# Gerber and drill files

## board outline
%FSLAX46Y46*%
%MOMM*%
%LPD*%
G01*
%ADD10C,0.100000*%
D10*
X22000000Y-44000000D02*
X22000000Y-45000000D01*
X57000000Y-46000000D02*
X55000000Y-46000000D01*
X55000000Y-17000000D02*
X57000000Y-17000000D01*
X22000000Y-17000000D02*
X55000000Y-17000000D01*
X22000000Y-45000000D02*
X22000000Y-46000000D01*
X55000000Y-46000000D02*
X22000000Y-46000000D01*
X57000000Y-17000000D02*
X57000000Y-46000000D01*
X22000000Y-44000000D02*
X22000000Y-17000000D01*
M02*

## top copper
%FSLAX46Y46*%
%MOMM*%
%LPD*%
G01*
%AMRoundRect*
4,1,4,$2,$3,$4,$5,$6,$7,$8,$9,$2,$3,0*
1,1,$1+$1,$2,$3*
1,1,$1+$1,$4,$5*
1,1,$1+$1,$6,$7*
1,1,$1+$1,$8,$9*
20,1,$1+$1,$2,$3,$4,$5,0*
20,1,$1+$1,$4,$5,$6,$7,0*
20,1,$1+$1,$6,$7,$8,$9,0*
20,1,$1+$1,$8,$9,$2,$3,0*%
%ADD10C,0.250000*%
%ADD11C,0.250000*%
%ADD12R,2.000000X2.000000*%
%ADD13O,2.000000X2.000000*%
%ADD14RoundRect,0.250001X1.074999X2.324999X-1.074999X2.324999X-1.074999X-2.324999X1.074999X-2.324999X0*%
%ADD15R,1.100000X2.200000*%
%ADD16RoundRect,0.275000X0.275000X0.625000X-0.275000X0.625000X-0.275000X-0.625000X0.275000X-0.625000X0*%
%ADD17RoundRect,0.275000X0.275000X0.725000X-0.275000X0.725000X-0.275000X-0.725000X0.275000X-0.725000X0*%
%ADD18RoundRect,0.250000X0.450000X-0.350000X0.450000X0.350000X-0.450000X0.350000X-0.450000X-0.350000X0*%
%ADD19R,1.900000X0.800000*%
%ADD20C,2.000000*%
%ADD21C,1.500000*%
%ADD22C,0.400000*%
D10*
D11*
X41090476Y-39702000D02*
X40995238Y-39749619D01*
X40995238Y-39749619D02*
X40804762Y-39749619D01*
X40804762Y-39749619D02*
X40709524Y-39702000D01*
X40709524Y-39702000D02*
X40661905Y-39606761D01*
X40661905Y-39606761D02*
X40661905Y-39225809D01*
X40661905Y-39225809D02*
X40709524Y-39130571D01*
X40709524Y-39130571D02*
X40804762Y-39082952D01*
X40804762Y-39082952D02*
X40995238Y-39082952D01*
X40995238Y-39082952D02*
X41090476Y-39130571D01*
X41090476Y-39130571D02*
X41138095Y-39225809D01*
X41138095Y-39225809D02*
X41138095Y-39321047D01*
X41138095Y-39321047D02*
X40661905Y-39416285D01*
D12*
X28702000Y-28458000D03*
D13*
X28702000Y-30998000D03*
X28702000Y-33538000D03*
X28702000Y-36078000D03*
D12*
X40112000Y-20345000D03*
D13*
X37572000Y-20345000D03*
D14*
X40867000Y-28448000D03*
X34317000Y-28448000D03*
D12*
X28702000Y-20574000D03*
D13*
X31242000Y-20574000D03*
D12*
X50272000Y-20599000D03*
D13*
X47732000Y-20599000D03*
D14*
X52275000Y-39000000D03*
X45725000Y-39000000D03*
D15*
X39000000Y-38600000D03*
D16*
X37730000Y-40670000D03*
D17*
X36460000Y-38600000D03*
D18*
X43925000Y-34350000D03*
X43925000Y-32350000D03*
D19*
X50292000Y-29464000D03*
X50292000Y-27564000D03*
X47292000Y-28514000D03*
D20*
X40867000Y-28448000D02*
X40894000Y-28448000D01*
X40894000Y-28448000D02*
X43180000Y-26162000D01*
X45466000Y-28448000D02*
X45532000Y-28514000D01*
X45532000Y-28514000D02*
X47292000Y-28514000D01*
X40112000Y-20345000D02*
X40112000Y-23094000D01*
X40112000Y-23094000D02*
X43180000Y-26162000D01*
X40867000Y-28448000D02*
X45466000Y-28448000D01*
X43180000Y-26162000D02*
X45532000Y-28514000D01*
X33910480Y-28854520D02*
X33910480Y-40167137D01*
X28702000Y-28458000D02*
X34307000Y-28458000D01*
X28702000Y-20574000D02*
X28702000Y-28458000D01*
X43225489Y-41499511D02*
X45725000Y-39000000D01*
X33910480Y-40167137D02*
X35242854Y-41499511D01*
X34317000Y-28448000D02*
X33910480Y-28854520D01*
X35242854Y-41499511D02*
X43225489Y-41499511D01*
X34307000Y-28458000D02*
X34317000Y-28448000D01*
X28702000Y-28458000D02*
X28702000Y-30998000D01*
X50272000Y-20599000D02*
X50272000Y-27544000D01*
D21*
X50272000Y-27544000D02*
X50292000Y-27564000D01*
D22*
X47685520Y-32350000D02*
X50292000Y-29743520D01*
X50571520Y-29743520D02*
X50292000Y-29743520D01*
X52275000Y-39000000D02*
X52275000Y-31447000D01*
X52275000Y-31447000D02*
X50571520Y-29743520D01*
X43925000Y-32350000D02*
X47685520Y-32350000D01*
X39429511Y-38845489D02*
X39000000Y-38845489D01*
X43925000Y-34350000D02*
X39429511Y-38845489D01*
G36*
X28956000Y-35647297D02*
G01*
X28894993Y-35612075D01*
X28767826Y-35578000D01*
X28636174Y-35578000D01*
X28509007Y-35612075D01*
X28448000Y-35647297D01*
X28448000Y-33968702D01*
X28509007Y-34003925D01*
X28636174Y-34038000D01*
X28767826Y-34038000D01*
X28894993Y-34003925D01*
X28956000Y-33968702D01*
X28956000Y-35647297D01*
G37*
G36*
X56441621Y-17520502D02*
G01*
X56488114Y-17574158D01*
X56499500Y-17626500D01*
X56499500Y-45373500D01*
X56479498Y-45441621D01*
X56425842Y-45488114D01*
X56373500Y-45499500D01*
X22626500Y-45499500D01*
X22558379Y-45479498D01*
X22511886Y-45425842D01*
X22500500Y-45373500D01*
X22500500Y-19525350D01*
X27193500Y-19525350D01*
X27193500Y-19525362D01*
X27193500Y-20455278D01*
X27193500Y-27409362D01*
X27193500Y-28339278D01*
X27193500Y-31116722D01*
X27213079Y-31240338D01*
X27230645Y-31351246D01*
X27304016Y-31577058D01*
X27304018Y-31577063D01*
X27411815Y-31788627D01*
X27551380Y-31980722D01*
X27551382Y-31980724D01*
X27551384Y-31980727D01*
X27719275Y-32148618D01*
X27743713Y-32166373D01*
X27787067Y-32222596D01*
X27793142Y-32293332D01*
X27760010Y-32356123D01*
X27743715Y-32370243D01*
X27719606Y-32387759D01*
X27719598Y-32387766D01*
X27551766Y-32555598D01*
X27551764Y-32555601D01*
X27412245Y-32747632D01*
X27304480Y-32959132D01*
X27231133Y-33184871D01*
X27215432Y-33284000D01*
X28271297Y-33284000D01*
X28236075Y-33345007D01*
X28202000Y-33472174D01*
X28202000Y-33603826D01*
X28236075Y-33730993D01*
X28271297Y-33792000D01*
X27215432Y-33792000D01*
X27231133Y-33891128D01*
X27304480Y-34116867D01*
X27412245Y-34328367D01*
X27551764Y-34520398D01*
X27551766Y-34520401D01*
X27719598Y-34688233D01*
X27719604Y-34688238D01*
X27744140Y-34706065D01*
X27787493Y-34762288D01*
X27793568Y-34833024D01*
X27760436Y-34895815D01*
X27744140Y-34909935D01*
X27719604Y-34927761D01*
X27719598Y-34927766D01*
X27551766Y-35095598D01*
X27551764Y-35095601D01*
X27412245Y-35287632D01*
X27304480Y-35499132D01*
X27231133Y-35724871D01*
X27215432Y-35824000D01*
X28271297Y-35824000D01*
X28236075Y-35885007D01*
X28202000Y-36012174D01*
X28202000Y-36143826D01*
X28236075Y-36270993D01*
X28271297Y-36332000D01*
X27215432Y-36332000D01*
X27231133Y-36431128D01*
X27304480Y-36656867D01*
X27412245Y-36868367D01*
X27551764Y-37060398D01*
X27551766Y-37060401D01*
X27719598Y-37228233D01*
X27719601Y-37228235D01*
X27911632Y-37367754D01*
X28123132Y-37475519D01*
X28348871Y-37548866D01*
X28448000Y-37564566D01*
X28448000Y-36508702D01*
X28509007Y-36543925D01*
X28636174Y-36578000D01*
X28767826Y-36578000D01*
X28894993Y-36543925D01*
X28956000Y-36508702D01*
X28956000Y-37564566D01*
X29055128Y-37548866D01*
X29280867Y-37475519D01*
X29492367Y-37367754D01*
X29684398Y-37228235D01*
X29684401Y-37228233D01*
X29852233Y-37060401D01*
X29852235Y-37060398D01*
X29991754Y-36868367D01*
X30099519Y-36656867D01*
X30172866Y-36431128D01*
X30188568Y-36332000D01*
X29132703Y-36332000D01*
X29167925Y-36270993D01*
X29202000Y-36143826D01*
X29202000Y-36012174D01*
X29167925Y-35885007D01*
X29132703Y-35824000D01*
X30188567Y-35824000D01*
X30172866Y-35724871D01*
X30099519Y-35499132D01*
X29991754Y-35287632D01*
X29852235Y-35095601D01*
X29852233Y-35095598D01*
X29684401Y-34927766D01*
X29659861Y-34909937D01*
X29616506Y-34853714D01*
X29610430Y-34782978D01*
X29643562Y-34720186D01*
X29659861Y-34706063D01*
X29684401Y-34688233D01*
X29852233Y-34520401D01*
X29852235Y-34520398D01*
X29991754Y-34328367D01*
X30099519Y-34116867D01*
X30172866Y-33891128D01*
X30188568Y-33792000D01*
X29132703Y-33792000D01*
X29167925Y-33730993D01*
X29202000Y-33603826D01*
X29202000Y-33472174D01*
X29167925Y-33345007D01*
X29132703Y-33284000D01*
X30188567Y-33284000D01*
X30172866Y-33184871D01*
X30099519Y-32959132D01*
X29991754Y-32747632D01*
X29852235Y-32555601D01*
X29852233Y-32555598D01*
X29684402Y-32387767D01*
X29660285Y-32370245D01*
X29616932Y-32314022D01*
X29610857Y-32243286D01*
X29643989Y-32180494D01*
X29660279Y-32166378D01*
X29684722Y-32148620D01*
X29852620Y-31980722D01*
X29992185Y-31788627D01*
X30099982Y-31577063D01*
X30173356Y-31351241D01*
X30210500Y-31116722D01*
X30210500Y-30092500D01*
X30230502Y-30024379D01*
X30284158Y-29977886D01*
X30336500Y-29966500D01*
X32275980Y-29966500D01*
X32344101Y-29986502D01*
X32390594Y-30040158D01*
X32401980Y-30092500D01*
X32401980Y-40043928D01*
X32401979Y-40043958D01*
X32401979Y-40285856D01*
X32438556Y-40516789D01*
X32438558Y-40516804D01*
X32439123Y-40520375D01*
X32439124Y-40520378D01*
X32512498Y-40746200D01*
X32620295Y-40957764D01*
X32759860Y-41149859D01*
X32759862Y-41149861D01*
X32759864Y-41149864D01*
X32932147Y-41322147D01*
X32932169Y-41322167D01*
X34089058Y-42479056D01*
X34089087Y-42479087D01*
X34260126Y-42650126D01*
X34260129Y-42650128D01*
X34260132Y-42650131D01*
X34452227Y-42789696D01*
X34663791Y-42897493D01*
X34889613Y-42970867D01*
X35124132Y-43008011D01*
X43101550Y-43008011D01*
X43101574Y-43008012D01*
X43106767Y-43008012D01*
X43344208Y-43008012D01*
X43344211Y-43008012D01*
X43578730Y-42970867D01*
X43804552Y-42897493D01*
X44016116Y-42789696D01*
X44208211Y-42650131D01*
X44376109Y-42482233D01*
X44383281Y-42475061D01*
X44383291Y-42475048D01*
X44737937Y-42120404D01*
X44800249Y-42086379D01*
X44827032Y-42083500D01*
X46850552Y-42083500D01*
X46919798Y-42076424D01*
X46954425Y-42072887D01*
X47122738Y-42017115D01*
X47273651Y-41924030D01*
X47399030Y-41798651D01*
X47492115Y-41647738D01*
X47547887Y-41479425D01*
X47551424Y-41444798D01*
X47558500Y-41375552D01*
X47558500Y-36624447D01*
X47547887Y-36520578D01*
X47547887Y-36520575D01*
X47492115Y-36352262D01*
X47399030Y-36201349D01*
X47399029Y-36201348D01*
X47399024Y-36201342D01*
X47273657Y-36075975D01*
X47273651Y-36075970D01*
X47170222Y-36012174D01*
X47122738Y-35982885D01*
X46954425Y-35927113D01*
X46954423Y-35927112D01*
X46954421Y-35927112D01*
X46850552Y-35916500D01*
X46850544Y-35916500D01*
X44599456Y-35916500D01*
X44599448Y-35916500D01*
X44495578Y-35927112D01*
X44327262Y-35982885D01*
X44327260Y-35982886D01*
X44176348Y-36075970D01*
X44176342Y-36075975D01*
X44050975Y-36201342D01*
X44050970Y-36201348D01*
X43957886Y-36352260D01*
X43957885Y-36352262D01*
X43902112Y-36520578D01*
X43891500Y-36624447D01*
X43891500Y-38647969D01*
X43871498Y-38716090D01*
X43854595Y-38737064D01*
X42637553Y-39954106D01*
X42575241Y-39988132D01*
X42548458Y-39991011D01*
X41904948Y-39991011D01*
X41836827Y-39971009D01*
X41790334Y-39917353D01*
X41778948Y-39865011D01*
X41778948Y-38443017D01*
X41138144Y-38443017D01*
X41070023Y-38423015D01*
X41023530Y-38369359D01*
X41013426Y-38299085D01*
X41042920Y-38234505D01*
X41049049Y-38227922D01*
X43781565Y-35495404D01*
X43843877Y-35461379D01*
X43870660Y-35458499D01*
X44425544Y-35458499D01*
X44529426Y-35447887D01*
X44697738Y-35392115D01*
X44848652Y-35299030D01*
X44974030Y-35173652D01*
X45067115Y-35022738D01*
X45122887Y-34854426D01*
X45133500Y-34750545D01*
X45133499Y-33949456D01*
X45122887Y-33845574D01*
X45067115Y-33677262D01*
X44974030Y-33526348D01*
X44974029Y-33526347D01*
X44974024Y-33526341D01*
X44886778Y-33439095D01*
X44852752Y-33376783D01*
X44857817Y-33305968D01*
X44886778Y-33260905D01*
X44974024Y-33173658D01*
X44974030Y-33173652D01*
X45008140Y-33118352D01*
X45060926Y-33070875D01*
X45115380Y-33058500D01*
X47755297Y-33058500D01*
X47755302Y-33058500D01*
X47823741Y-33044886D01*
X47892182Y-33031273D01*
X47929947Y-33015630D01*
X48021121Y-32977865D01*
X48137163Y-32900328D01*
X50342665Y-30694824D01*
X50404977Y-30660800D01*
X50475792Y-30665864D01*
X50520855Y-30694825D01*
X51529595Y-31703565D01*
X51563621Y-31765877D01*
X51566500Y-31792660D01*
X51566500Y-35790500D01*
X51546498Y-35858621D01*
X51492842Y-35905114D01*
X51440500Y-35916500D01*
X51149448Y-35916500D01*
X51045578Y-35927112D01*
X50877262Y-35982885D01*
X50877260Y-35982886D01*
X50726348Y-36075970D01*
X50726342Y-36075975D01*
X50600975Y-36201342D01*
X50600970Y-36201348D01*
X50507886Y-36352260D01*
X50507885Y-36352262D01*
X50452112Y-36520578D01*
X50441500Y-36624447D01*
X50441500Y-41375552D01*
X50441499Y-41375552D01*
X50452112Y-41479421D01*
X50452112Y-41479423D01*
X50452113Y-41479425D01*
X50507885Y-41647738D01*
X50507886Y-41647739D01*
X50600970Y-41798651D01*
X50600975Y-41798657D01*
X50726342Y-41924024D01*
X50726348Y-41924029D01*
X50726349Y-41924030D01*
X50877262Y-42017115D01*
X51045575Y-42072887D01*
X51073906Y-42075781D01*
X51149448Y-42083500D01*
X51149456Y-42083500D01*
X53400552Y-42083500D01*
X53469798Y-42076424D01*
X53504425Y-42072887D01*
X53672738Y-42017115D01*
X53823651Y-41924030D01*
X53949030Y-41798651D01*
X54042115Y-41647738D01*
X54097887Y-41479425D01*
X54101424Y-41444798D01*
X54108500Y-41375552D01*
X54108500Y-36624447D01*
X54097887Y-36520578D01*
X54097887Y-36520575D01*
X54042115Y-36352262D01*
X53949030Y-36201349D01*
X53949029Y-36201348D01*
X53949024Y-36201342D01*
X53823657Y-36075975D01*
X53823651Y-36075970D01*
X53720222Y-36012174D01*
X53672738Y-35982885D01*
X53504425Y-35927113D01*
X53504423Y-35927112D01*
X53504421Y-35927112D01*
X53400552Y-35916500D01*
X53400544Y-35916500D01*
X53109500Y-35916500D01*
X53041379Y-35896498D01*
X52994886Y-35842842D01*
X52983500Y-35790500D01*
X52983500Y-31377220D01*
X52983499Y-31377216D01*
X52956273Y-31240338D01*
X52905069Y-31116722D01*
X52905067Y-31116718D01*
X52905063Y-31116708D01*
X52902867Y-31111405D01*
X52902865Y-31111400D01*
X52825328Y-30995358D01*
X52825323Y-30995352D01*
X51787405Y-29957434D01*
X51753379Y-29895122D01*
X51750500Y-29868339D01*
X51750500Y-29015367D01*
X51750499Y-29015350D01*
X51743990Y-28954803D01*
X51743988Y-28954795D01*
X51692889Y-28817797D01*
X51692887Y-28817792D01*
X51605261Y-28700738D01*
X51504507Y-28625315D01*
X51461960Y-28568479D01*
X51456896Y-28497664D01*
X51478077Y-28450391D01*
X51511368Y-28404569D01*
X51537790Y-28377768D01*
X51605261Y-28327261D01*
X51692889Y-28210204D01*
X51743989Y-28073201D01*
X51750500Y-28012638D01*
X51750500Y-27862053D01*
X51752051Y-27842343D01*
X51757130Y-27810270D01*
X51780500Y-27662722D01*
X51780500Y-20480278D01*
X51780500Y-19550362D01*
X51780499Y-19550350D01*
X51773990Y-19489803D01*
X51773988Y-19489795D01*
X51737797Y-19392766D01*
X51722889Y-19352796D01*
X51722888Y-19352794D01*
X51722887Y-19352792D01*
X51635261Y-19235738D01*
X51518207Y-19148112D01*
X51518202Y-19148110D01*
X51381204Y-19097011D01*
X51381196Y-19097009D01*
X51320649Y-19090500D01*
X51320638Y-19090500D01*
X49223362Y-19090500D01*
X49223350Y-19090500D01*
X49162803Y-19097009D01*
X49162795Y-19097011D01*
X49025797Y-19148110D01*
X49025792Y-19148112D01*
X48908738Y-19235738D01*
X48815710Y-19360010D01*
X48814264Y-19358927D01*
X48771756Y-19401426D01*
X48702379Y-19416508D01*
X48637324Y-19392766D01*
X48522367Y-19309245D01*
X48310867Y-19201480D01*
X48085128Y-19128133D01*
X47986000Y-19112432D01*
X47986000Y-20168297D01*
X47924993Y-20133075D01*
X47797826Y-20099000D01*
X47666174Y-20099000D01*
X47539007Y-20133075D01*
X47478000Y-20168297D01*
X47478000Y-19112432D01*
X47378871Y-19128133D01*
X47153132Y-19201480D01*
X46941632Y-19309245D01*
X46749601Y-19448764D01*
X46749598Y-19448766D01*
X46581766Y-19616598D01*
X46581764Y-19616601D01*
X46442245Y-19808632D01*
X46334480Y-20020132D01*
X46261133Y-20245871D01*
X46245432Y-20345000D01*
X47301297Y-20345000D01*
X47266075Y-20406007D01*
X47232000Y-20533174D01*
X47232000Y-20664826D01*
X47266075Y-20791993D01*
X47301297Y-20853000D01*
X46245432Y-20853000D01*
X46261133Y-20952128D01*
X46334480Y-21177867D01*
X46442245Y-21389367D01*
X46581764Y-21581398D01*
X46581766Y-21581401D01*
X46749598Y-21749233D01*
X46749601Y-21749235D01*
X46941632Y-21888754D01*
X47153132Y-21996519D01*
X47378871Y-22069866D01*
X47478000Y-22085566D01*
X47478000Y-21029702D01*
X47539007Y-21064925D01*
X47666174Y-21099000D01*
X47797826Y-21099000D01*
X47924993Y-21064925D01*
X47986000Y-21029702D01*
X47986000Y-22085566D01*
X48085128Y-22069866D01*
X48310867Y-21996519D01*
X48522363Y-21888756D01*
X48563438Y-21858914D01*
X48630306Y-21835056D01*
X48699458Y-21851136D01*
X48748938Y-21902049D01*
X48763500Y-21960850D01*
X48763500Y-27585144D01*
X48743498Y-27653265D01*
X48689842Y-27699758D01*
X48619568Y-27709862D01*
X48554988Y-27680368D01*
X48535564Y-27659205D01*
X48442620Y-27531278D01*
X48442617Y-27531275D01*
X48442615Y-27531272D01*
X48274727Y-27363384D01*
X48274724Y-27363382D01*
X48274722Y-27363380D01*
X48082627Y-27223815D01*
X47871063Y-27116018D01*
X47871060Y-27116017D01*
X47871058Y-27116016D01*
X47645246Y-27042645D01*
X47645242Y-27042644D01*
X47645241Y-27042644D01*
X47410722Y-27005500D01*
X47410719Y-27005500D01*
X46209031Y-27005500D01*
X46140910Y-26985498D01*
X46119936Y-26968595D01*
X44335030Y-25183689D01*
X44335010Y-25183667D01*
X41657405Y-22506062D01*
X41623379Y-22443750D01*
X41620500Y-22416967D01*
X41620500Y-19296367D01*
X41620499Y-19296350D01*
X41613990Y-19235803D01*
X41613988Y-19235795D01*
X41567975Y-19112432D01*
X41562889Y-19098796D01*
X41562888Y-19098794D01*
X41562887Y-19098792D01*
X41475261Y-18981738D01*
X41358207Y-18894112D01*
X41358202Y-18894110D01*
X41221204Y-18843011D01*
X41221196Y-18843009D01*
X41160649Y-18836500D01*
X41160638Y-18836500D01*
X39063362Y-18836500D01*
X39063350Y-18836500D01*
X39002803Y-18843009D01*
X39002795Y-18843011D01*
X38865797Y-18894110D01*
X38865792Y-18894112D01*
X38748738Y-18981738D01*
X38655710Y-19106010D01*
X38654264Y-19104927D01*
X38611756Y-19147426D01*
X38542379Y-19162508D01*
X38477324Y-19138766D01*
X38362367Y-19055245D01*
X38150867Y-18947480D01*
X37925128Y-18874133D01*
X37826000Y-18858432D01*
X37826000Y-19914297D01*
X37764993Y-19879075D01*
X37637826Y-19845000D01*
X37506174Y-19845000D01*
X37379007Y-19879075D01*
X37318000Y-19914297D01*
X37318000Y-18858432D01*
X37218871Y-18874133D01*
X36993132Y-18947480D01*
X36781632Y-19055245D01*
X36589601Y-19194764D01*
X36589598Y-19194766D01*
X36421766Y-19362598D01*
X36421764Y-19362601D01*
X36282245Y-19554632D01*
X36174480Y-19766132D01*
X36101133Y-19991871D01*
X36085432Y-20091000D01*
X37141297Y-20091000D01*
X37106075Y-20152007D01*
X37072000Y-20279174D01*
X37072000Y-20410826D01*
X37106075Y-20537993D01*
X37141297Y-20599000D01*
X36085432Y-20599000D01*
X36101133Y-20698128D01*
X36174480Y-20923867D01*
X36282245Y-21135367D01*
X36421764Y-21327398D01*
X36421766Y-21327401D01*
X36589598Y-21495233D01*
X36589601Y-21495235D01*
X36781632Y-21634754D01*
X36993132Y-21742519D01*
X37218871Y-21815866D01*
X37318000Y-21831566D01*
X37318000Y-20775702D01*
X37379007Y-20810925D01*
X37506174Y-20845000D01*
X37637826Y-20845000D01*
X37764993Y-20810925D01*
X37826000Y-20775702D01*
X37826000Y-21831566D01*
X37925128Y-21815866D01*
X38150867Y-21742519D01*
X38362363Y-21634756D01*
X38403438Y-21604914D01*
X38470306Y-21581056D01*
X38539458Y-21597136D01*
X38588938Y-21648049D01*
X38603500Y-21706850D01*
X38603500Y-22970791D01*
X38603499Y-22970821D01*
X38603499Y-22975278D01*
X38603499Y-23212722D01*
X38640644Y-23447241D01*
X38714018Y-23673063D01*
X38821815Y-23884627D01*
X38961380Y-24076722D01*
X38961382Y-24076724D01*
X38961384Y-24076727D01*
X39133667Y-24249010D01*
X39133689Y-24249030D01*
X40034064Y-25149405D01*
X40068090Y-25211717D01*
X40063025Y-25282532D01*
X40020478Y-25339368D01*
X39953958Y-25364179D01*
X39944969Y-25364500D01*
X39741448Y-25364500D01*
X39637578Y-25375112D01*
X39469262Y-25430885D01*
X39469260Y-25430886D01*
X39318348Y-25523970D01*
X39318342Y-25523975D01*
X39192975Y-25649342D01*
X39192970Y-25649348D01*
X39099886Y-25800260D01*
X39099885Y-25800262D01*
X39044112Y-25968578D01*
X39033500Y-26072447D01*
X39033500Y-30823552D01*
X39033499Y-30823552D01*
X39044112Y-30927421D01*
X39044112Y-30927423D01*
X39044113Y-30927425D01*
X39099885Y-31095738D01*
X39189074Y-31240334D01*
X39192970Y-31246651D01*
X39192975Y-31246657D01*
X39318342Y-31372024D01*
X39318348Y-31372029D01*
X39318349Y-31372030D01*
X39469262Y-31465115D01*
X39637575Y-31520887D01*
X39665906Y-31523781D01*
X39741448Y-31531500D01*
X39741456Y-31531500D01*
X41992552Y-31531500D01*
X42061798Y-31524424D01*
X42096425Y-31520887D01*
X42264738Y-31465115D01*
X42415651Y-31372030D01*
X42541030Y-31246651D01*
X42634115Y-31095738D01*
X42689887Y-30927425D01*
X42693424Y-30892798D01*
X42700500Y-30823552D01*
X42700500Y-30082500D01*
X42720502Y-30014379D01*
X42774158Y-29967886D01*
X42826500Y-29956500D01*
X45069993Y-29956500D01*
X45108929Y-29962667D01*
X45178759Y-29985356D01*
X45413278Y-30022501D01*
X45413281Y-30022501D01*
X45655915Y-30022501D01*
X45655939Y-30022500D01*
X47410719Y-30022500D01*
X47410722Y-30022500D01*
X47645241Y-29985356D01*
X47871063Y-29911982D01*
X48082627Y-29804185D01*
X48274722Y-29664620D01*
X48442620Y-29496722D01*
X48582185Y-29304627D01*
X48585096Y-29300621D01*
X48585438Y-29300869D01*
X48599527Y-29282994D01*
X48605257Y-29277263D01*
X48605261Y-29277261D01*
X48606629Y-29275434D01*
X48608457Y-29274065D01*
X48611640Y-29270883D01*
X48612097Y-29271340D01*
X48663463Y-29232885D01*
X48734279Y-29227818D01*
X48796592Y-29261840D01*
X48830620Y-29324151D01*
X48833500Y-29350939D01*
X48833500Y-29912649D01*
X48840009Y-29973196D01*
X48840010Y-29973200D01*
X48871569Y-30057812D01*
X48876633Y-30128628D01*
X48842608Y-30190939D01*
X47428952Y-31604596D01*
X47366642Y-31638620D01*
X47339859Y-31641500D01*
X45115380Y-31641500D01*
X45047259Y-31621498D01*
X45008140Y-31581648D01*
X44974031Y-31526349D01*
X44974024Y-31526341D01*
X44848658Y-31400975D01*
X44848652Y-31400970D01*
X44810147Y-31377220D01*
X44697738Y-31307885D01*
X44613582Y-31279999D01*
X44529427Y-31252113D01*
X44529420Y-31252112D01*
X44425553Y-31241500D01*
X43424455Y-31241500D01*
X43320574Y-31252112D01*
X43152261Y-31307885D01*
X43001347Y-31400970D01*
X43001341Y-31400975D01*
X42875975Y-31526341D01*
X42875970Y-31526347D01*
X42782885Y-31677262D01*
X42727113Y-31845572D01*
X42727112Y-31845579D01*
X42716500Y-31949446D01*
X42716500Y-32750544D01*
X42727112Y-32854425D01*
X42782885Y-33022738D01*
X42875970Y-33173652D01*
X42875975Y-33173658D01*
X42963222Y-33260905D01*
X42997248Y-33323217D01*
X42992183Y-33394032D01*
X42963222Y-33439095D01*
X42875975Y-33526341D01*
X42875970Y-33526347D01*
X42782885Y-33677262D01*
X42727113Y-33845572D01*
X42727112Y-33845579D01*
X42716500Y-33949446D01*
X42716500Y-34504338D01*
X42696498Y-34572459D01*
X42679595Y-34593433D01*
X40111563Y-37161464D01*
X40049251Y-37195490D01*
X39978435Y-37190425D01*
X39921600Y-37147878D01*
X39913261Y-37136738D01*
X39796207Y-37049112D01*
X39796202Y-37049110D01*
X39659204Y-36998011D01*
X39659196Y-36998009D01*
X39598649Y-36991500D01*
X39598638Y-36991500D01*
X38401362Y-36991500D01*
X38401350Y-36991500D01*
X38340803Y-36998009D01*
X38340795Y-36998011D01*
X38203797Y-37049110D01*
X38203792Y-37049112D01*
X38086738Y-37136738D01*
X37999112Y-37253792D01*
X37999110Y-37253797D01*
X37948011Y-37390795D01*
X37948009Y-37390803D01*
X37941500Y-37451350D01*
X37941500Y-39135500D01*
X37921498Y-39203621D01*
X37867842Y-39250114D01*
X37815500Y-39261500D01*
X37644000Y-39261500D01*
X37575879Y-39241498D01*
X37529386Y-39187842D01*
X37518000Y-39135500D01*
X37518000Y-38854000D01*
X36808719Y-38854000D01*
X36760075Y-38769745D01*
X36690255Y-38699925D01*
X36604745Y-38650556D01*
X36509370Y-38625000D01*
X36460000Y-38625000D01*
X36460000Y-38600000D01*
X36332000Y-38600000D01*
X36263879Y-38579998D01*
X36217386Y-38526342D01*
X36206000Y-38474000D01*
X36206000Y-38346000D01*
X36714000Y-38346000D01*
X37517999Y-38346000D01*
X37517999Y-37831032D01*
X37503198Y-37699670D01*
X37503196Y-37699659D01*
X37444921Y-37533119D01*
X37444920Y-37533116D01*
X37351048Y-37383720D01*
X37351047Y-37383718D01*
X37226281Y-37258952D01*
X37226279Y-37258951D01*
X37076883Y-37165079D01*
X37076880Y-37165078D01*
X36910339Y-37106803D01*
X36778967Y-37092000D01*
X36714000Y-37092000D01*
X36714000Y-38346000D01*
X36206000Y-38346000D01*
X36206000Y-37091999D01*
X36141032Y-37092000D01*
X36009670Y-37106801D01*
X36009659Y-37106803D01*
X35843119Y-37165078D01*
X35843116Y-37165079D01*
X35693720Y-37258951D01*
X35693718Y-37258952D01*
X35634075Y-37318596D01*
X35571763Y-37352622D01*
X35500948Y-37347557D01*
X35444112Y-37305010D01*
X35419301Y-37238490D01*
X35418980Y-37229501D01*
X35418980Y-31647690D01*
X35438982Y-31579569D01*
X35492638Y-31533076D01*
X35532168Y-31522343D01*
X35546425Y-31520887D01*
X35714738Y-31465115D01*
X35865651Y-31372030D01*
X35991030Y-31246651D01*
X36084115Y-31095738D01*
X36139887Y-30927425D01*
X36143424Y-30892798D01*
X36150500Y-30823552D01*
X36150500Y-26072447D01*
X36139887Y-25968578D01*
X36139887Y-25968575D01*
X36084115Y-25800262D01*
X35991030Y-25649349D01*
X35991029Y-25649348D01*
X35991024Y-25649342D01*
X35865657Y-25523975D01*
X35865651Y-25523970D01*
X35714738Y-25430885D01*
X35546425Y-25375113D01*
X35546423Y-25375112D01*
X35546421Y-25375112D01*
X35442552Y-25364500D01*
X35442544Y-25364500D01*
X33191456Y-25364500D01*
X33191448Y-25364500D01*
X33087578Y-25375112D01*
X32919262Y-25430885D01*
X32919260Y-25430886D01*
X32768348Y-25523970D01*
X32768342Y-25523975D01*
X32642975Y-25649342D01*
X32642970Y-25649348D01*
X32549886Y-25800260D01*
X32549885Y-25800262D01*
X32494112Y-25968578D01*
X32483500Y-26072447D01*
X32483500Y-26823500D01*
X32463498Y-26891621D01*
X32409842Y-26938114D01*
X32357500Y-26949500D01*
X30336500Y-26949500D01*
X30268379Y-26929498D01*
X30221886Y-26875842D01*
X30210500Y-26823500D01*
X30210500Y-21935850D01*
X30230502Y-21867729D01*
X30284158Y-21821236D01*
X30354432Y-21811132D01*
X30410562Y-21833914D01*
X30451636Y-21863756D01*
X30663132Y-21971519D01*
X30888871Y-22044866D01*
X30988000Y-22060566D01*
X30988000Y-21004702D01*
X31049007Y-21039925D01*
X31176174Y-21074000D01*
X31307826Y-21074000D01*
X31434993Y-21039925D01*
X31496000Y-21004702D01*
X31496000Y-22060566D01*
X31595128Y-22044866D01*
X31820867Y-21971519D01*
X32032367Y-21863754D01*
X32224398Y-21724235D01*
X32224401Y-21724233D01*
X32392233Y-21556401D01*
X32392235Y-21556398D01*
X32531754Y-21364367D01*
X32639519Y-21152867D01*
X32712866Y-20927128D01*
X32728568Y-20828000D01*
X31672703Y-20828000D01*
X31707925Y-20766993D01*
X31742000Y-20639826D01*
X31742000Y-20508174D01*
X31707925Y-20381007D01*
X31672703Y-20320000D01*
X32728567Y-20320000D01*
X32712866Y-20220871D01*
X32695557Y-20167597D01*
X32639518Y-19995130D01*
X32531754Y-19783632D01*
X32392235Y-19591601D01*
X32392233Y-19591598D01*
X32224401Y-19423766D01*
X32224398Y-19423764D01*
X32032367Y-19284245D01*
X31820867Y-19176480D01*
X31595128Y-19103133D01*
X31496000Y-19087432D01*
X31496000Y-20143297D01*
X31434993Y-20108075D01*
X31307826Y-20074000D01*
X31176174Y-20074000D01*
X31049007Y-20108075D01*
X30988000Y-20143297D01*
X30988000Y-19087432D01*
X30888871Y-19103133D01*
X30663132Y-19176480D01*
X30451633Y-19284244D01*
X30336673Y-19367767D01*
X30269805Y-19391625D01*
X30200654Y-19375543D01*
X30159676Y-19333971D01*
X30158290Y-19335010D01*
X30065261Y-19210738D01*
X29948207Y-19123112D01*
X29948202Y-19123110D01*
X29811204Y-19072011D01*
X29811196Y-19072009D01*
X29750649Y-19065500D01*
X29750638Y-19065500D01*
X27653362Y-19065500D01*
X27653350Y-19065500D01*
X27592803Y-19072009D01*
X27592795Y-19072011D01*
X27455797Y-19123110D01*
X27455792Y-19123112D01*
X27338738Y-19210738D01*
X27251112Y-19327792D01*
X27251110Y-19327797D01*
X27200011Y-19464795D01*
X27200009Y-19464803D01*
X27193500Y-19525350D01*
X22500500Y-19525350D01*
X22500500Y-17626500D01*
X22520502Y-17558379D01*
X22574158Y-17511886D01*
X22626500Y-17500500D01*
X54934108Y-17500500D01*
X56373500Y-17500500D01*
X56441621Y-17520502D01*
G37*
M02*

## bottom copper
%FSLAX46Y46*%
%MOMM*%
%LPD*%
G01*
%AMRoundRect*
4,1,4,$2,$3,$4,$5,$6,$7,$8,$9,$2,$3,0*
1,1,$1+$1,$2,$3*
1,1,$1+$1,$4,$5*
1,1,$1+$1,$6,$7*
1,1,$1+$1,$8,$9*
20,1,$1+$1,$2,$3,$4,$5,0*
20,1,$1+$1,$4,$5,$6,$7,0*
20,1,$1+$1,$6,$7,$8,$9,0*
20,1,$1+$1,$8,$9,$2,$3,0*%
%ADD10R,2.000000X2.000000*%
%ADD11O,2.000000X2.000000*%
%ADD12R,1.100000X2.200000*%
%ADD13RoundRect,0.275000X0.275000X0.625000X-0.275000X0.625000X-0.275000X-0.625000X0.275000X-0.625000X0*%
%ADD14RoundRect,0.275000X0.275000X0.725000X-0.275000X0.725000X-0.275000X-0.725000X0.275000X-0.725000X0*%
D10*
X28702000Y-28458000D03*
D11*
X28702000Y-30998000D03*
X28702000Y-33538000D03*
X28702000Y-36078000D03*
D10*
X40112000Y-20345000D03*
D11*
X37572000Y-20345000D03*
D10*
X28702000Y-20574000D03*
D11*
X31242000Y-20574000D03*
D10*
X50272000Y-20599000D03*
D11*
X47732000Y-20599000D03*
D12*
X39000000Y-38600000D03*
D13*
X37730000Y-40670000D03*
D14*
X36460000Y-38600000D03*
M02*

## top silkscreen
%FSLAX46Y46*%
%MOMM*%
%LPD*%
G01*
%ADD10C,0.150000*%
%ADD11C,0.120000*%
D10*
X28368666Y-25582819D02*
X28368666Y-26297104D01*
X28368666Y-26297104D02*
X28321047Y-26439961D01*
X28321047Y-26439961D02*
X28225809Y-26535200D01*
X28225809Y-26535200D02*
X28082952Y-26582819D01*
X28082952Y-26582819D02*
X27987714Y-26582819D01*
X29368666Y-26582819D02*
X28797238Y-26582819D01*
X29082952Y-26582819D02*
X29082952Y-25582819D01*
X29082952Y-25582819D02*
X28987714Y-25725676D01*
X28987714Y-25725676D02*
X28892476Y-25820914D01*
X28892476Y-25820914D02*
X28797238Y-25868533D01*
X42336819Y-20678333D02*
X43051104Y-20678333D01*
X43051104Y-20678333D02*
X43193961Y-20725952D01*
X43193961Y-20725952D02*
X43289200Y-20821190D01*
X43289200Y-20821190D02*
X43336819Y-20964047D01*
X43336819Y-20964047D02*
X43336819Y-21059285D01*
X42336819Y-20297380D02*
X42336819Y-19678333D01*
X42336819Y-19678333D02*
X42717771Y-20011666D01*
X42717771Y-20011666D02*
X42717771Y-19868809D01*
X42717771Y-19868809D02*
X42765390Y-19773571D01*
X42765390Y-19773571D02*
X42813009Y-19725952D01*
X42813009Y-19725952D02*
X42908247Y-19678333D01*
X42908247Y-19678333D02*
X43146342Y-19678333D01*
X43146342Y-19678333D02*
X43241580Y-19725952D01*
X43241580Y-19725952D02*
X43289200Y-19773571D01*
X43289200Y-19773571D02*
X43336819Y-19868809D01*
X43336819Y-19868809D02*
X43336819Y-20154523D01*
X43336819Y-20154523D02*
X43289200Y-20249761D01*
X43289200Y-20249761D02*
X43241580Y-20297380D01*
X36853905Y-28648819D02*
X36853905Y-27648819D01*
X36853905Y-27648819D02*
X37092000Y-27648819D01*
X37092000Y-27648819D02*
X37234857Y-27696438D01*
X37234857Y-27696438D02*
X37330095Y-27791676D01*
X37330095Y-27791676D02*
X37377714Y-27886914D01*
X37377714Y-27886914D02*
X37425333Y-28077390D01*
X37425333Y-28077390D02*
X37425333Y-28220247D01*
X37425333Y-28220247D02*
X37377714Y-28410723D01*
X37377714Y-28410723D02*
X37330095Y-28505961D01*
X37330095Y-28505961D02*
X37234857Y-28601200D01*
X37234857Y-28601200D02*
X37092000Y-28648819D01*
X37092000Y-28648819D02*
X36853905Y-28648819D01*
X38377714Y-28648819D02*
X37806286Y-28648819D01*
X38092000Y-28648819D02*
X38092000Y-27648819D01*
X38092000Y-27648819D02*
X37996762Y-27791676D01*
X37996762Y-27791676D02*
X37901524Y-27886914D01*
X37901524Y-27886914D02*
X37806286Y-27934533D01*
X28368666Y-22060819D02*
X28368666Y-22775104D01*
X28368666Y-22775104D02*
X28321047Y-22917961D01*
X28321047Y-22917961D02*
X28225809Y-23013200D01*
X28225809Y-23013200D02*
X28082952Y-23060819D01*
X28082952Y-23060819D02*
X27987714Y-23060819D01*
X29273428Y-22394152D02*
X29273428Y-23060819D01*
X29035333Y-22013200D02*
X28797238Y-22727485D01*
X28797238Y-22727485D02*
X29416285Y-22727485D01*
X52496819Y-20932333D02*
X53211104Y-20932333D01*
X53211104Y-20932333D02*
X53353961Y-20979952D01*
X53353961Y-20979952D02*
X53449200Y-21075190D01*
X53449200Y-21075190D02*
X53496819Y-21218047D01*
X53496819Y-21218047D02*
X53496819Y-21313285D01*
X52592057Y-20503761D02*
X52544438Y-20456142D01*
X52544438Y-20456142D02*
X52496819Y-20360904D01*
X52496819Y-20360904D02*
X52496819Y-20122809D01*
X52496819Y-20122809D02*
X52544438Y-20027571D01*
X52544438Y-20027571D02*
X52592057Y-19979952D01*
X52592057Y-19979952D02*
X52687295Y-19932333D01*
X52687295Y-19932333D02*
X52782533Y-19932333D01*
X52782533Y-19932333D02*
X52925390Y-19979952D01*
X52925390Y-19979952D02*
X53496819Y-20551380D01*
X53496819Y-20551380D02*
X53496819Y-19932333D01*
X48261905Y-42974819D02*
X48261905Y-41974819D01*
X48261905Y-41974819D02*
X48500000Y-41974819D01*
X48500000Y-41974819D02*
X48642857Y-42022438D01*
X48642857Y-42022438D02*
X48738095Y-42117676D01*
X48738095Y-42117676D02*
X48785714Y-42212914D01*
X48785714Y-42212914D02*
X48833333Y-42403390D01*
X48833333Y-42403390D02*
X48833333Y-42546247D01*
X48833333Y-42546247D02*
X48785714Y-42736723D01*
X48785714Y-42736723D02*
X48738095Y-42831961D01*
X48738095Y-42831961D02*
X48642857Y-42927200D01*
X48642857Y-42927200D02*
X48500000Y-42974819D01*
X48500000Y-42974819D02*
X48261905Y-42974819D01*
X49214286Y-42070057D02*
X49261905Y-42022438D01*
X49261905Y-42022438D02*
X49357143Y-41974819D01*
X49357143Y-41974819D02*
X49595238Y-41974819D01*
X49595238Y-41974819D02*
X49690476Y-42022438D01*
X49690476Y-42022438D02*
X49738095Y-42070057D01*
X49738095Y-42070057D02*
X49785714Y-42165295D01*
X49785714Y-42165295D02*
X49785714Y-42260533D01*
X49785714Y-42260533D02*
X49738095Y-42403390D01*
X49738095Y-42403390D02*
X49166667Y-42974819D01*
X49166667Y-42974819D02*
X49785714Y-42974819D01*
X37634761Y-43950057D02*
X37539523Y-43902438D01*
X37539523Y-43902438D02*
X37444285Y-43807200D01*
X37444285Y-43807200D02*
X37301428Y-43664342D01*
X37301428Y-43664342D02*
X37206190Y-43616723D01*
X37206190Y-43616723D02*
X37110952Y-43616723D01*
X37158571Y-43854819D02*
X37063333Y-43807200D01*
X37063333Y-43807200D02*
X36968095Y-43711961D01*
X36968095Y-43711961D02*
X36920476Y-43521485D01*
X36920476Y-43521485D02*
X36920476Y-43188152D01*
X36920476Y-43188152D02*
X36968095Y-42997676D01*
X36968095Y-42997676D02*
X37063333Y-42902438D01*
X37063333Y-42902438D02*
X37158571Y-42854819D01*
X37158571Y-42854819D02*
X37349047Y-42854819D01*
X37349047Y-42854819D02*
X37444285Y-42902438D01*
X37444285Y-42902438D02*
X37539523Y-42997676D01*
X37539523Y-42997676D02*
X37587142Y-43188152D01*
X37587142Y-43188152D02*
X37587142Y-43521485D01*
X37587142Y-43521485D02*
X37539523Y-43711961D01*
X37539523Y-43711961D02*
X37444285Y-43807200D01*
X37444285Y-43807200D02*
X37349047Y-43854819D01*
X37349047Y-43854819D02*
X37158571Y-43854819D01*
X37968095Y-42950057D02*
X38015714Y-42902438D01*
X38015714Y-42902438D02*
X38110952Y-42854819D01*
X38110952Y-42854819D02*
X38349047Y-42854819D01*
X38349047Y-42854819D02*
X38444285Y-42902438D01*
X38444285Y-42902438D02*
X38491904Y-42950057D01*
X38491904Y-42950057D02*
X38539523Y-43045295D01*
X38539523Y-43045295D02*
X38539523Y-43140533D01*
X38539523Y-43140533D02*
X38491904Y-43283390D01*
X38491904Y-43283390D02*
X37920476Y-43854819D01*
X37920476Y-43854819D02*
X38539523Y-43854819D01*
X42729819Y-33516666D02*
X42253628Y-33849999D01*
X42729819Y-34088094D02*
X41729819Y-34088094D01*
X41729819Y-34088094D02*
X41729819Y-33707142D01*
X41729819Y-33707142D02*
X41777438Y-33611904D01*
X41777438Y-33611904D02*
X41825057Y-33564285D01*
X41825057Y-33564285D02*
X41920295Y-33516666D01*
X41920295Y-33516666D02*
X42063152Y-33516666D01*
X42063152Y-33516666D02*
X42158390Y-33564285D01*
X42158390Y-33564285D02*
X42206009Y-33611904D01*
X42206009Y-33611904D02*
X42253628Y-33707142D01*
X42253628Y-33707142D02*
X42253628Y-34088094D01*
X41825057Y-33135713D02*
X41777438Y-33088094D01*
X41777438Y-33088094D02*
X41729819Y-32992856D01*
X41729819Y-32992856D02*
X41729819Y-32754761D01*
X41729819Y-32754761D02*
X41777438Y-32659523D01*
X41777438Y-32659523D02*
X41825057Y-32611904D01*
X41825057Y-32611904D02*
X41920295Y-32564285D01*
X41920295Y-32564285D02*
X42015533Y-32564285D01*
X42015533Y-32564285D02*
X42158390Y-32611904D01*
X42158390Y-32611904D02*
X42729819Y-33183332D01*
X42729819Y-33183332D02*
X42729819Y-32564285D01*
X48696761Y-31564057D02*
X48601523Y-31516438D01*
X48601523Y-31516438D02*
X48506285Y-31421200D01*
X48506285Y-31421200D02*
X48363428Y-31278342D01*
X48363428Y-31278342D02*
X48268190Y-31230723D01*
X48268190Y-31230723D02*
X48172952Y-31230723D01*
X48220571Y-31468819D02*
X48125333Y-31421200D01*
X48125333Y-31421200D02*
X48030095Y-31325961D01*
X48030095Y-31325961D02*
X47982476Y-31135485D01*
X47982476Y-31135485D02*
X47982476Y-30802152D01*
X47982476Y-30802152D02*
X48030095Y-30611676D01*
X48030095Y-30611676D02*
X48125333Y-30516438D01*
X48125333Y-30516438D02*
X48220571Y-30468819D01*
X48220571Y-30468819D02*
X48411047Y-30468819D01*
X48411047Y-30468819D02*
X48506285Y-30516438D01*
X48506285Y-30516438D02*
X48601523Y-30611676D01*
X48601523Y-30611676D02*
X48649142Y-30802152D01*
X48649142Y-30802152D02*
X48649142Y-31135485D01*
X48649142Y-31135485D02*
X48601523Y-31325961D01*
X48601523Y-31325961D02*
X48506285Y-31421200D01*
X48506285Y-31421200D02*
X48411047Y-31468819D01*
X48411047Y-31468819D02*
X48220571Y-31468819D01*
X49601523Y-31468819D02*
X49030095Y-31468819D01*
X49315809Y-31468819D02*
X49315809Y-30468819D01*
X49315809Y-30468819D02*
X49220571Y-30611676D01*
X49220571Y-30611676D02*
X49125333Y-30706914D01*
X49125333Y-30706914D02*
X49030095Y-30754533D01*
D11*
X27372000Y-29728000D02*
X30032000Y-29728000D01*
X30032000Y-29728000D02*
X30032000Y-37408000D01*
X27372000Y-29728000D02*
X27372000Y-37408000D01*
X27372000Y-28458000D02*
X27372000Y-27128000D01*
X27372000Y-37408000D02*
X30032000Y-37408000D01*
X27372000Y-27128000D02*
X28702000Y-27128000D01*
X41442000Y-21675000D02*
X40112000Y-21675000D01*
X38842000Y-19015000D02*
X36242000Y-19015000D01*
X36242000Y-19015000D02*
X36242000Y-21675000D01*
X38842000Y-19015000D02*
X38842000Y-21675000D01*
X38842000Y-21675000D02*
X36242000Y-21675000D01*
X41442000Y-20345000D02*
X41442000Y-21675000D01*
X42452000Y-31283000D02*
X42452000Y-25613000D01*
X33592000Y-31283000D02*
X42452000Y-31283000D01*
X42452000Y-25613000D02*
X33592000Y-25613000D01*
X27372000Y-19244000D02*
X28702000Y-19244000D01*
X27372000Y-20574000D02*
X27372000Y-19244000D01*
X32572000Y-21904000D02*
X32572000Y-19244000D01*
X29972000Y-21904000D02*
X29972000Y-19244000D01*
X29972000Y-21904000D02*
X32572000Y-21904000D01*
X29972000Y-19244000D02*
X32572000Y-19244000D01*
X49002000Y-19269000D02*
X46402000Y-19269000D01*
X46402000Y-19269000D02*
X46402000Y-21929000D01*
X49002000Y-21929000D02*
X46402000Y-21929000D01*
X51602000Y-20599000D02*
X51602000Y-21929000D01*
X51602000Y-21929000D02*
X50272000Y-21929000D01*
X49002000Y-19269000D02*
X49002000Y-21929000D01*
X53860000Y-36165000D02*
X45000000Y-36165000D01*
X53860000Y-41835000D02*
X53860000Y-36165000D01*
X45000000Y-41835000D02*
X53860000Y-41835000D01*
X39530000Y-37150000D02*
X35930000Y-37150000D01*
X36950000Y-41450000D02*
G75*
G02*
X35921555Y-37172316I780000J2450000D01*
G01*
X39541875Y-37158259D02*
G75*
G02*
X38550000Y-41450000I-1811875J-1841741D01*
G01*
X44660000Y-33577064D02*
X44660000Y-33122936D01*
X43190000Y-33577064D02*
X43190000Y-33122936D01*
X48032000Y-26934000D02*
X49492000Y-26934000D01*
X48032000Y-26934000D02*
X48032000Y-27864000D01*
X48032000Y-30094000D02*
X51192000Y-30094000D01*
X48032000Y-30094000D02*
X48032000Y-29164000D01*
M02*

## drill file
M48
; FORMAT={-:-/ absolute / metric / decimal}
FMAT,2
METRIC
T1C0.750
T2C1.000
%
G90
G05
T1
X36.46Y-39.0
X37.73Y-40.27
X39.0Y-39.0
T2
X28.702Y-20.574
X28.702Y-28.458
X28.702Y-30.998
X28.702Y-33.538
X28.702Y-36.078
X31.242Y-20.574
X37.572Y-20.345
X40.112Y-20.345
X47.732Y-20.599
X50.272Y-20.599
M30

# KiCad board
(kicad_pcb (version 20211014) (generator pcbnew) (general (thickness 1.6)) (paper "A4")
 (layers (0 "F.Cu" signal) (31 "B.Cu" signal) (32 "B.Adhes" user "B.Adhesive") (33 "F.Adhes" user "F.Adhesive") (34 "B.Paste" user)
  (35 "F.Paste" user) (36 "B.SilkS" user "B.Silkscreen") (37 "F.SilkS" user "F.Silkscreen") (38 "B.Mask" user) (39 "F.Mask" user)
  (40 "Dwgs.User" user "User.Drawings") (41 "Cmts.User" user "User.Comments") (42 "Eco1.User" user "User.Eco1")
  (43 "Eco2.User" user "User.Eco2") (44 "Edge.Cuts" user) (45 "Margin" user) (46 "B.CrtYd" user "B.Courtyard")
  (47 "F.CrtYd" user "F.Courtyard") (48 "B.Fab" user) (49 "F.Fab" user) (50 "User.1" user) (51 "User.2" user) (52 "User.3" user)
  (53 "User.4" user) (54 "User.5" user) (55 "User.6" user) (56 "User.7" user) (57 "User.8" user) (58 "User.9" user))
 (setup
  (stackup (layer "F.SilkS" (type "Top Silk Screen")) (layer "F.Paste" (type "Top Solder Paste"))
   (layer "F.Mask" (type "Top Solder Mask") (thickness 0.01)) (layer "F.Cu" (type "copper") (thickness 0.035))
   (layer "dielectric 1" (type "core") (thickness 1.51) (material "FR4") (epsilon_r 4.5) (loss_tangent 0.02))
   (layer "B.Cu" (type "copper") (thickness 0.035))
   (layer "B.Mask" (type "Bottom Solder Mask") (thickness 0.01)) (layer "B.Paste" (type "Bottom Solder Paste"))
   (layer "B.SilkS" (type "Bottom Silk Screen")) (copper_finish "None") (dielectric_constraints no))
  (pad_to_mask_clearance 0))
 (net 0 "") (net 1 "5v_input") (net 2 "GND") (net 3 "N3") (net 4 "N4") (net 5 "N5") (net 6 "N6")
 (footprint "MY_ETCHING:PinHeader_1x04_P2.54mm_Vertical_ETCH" (layer "F.Cu") (at 28.702 28.458)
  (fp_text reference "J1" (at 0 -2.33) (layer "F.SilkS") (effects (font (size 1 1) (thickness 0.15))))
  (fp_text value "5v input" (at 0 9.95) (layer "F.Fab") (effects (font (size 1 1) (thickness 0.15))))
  (fp_line (start -1.33 1.27) (end 1.33 1.27) (layer "F.SilkS") (width 0.12))
  (fp_line (start 1.33 1.27) (end 1.33 8.95) (layer "F.SilkS") (width 0.12))
  (fp_line (start -1.33 1.27) (end -1.33 8.95) (layer "F.SilkS") (width 0.12))
  (fp_line (start -1.33 0) (end -1.33 -1.33) (layer "F.SilkS") (width 0.12))
  (fp_line (start -1.33 8.95) (end 1.33 8.95) (layer "F.SilkS") (width 0.12))
  (fp_line (start -1.33 -1.33) (end 0 -1.33) (layer "F.SilkS") (width 0.12))
  (pad "1" thru_hole rect (at 0 0) (size 2 2) (drill 1) (layers *.Cu *.Mask) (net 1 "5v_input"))
  (pad "2" thru_hole oval (at 0 2.54) (size 2 2) (drill 1) (layers *.Cu *.Mask) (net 1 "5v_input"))
  (pad "3" thru_hole oval (at 0 5.08) (size 2 2) (drill 1) (layers *.Cu *.Mask) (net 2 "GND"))
  (pad "4" thru_hole oval (at 0 7.62) (size 2 2) (drill 1) (layers *.Cu *.Mask) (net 2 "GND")))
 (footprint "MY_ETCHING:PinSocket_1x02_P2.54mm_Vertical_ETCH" (layer "F.Cu") (at 40.112 20.345 -90)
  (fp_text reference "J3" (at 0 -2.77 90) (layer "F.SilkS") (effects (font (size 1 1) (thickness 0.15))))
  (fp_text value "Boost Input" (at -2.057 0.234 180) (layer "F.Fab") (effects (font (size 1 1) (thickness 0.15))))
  (fp_line (start 1.33 -1.33) (end 1.33 0) (layer "F.SilkS") (width 0.12))
  (fp_line (start -1.33 1.27) (end -1.33 3.87) (layer "F.SilkS") (width 0.12))
  (fp_line (start -1.33 3.87) (end 1.33 3.87) (layer "F.SilkS") (width 0.12))
  (fp_line (start -1.33 1.27) (end 1.33 1.27) (layer "F.SilkS") (width 0.12))
  (fp_line (start 1.33 1.27) (end 1.33 3.87) (layer "F.SilkS") (width 0.12))
  (fp_line (start 0 -1.33) (end 1.33 -1.33) (layer "F.SilkS") (width 0.12))
  (pad "1" thru_hole rect (at 0 0 270) (size 2 2) (drill 1) (layers *.Cu *.Mask) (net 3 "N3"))
  (pad "2" thru_hole oval (at 0 2.54 270) (size 2 2) (drill 1) (layers *.Cu *.Mask) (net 2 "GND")))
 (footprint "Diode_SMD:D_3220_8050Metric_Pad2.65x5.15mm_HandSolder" (layer "F.Cu") (at 37.592 28.448 180)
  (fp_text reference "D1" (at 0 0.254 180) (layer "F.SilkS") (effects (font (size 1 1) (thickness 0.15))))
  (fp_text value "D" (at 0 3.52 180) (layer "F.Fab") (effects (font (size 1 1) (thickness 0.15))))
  (fp_line (start -4.86 -2.835) (end -4.86 2.835) (layer "F.SilkS") (width 0.12))
  (fp_line (start 4 -2.835) (end -4.86 -2.835) (layer "F.SilkS") (width 0.12))
  (fp_line (start -4.86 2.835) (end 4 2.835) (layer "F.SilkS") (width 0.12))
  (pad "1" smd roundrect (at -3.275 0 180) (size 2.65 5.15) (layers "F.Cu" "F.Paste" "F.Mask") (roundrect_rratio 0.09434) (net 3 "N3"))
  (pad "2" smd roundrect (at 3.275 0 180) (size 2.65 5.15) (layers "F.Cu" "F.Paste" "F.Mask") (roundrect_rratio 0.09434) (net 1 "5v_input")))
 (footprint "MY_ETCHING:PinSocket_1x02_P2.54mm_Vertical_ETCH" (layer "F.Cu") (at 28.702 20.574 90)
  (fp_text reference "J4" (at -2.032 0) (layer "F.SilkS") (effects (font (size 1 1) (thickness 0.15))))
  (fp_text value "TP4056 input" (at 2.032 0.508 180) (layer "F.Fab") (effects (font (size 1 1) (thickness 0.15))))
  (fp_line (start 1.33 -1.33) (end 1.33 0) (layer "F.SilkS") (width 0.12))
  (fp_line (start 0 -1.33) (end 1.33 -1.33) (layer "F.SilkS") (width 0.12))
  (fp_line (start -1.33 3.87) (end 1.33 3.87) (layer "F.SilkS") (width 0.12))
  (fp_line (start -1.33 1.27) (end 1.33 1.27) (layer "F.SilkS") (width 0.12))
  (fp_line (start -1.33 1.27) (end -1.33 3.87) (layer "F.SilkS") (width 0.12))
  (fp_line (start 1.33 1.27) (end 1.33 3.87) (layer "F.SilkS") (width 0.12))
  (pad "1" thru_hole rect (at 0 0 90) (size 2 2) (drill 1) (layers *.Cu *.Mask) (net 1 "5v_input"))
  (pad "2" thru_hole oval (at 0 2.54 90) (size 2 2) (drill 1) (layers *.Cu *.Mask) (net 2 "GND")))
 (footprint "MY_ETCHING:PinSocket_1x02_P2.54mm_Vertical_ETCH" (layer "F.Cu") (at 50.272 20.599 -90)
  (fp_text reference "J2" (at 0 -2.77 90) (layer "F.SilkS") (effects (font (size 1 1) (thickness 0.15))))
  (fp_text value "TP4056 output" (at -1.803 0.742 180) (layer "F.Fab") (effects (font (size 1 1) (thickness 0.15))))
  (fp_line (start -1.33 1.27) (end -1.33 3.87) (layer "F.SilkS") (width 0.12))
  (fp_line (start -1.33 3.87) (end 1.33 3.87) (layer "F.SilkS") (width 0.12))
  (fp_line (start 1.33 1.27) (end 1.33 3.87) (layer "F.SilkS") (width 0.12))
  (fp_line (start 0 -1.33) (end 1.33 -1.33) (layer "F.SilkS") (width 0.12))
  (fp_line (start 1.33 -1.33) (end 1.33 0) (layer "F.SilkS") (width 0.12))
  (fp_line (start -1.33 1.27) (end 1.33 1.27) (layer "F.SilkS") (width 0.12))
  (pad "1" thru_hole rect (at 0 0 270) (size 2 2) (drill 1) (layers *.Cu *.Mask) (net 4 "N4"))
  (pad "2" thru_hole oval (at 0 2.54 270) (size 2 2) (drill 1) (layers *.Cu *.Mask) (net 2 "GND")))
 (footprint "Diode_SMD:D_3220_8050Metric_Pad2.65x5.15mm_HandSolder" (layer "F.Cu") (at 49 39 180)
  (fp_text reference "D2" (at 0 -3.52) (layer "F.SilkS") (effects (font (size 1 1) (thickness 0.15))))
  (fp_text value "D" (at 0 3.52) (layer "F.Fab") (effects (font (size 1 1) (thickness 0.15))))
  (fp_line (start -4.86 2.835) (end 4 2.835) (layer "F.SilkS") (width 0.12))
  (fp_line (start -4.86 -2.835) (end -4.86 2.835) (layer "F.SilkS") (width 0.12))
  (fp_line (start 4 -2.835) (end -4.86 -2.835) (layer "F.SilkS") (width 0.12))
  (pad "1" smd roundrect (at -3.275 0 180) (size 2.65 5.15) (layers "F.Cu" "F.Paste" "F.Mask") (roundrect_rratio 0.09434) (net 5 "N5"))
  (pad "2" smd roundrect (at 3.275 0 180) (size 2.65 5.15) (layers "F.Cu" "F.Paste" "F.Mask") (roundrect_rratio 0.09434) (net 1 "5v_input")))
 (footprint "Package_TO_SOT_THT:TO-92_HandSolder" (layer "F.Cu") (at 39 39 180)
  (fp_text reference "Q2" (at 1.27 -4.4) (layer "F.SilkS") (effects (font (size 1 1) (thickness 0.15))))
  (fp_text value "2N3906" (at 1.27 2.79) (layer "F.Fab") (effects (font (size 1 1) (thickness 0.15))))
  (fp_line (start -0.53 1.85) (end 3.07 1.85) (layer "F.SilkS") (width 0.12))
  (fp_arc (start 2.05 -2.45) (mid 3.769931 -0.601036) (end 3.078445 1.827684) (layer "F.SilkS") (width 0.12))
  (fp_arc (start -0.541875 1.841741) (mid -1.247231 -0.581764) (end 0.45 -2.45) (layer "F.SilkS") (width 0.12))
  (pad "1" thru_hole rect (at 0 0 180) (size 1.1 2.2) (drill 0.75 (offset 0 0.4)) (layers *.Cu *.Mask) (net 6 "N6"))
  (pad "2" thru_hole roundrect (at 1.27 -1.27 180) (size 1.1 1.8) (drill 0.75 (offset 0 -0.4)) (layers *.Cu *.Mask) (roundrect_rratio 0.25)
   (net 1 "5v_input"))
  (pad "3" thru_hole roundrect (at 2.54 0 180) (size 1.1 2) (drill 0.75 (offset 0 0.4)) (layers *.Cu *.Mask) (roundrect_rratio 0.25)
   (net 2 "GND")))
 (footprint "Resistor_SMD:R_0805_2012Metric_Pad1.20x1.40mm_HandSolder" (layer "F.Cu") (at 43.925 33.35 90)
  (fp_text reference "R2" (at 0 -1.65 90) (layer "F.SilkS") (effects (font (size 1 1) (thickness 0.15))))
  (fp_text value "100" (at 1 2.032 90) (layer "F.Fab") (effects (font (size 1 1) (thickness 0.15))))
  (fp_line (start -0.227064 0.735) (end 0.227064 0.735) (layer "F.SilkS") (width 0.12))
  (fp_line (start -0.227064 -0.735) (end 0.227064 -0.735) (layer "F.SilkS") (width 0.12))
  (pad "1" smd roundrect (at -1 0 90) (size 1.2 1.4) (layers "F.Cu" "F.Paste" "F.Mask") (roundrect_rratio 0.2083333333) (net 6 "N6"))
  (pad "2" smd roundrect (at 1 0 90) (size 1.2 1.4) (layers "F.Cu" "F.Paste" "F.Mask") (roundrect_rratio 0.2083333333) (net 5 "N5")))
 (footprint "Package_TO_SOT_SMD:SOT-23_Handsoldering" (layer "F.Cu") (at 48.792 28.514 180)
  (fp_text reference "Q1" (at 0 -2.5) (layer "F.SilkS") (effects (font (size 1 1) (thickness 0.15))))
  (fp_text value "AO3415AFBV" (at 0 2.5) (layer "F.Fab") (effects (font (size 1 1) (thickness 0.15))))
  (fp_line (start 0.76 1.58) (end -0.7 1.58) (layer "F.SilkS") (width 0.12))
  (fp_line (start 0.76 1.58) (end 0.76 0.65) (layer "F.SilkS") (width 0.12))
  (fp_line (start 0.76 -1.58) (end -2.4 -1.58) (layer "F.SilkS") (width 0.12))
  (fp_line (start 0.76 -1.58) (end 0.76 -0.65) (layer "F.SilkS") (width 0.12))
  (pad "1" smd rect (at -1.5 -0.95 180) (size 1.9 0.8) (layers "F.Cu" "F.Paste" "F.Mask") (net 5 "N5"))
  (pad "2" smd rect (at -1.5 0.95 180) (size 1.9 0.8) (layers "F.Cu" "F.Paste" "F.Mask") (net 4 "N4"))
  (pad "3" smd rect (at 1.5 0 180) (size 1.9 0.8) (layers "F.Cu" "F.Paste" "F.Mask") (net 3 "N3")))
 (gr_line (start 22 44) (end 22 45) (layer "Edge.Cuts") (width 0.1))
 (gr_line (start 57 46) (end 55 46) (layer "Edge.Cuts") (width 0.1))
 (gr_line (start 55 17) (end 57 17) (layer "Edge.Cuts") (width 0.1))
 (gr_line (start 22 17) (end 55 17) (layer "Edge.Cuts") (width 0.1))
 (gr_line (start 22 45) (end 22 46) (layer "Edge.Cuts") (width 0.1))
 (gr_line (start 55 46) (end 22 46) (layer "Edge.Cuts") (width 0.1))
 (gr_line (start 57 17) (end 57 46) (layer "Edge.Cuts") (width 0.1))
 (gr_line (start 22 44) (end 22 17) (layer "Edge.Cuts") (width 0.1))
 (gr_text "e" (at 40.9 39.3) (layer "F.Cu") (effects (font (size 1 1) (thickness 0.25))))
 (segment (start 40.867 28.448) (end 40.894 28.448) (width 2) (layer "F.Cu") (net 3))
 (segment (start 40.894 28.448) (end 43.18 26.162) (width 2) (layer "F.Cu") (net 3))
 (segment (start 45.466 28.448) (end 45.532 28.514) (width 2) (layer "F.Cu") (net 3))
 (segment (start 45.532 28.514) (end 47.292 28.514) (width 2) (layer "F.Cu") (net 3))
 (segment (start 40.112 20.345) (end 40.112 23.094) (width 2) (layer "F.Cu") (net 3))
 (segment (start 40.112 23.094) (end 43.18 26.162) (width 2) (layer "F.Cu") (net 3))
 (segment (start 40.867 28.448) (end 45.466 28.448) (width 2) (layer "F.Cu") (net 3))
 (segment (start 43.18 26.162) (end 45.532 28.514) (width 2) (layer "F.Cu") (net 3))
 (segment (start 33.91048 28.85452) (end 33.91048 40.167137) (width 2) (layer "F.Cu") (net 1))
 (segment (start 28.702 28.458) (end 34.307 28.458) (width 2) (layer "F.Cu") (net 1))
 (segment (start 28.702 20.574) (end 28.702 28.458) (width 2) (layer "F.Cu") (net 1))
 (segment (start 43.225489 41.499511) (end 45.725 39) (width 2) (layer "F.Cu") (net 1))
 (segment (start 33.91048 40.167137) (end 35.242854 41.499511) (width 2) (layer "F.Cu") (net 1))
 (segment (start 34.317 28.448) (end 33.91048 28.85452) (width 2) (layer "F.Cu") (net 1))
 (segment (start 35.242854 41.499511) (end 43.225489 41.499511) (width 2) (layer "F.Cu") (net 1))
 (segment (start 34.307 28.458) (end 34.317 28.448) (width 2) (layer "F.Cu") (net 1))
 (segment (start 28.702 28.458) (end 28.702 30.998) (width 2) (layer "F.Cu") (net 1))
 (segment (start 50.272 20.599) (end 50.272 27.544) (width 2) (layer "F.Cu") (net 4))
 (segment (start 50.272 27.544) (end 50.292 27.564) (width 1.5) (layer "F.Cu") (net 4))
 (segment (start 47.68552 32.35) (end 50.292 29.74352) (width 0.4) (layer "F.Cu") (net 5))
 (segment (start 50.57152 29.74352) (end 50.292 29.74352) (width 0.4) (layer "F.Cu") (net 5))
 (segment (start 52.275 39) (end 52.275 31.447) (width 0.4) (layer "F.Cu") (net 5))
 (segment (start 52.275 31.447) (end 50.57152 29.74352) (width 0.4) (layer "F.Cu") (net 5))
 (segment (start 43.925 32.35) (end 47.68552 32.35) (width 0.4) (layer "F.Cu") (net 5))
 (segment (start 39.429511 38.845489) (end 39 38.845489) (width 0.4) (layer "F.Cu") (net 6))
 (segment (start 43.925 34.35) (end 39.429511 38.845489) (width 0.4) (layer "F.Cu") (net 6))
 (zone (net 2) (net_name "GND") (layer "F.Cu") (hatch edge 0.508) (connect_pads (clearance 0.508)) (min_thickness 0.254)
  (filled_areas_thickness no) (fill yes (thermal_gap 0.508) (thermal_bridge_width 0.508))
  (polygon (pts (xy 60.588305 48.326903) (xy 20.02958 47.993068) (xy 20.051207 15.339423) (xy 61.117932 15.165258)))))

